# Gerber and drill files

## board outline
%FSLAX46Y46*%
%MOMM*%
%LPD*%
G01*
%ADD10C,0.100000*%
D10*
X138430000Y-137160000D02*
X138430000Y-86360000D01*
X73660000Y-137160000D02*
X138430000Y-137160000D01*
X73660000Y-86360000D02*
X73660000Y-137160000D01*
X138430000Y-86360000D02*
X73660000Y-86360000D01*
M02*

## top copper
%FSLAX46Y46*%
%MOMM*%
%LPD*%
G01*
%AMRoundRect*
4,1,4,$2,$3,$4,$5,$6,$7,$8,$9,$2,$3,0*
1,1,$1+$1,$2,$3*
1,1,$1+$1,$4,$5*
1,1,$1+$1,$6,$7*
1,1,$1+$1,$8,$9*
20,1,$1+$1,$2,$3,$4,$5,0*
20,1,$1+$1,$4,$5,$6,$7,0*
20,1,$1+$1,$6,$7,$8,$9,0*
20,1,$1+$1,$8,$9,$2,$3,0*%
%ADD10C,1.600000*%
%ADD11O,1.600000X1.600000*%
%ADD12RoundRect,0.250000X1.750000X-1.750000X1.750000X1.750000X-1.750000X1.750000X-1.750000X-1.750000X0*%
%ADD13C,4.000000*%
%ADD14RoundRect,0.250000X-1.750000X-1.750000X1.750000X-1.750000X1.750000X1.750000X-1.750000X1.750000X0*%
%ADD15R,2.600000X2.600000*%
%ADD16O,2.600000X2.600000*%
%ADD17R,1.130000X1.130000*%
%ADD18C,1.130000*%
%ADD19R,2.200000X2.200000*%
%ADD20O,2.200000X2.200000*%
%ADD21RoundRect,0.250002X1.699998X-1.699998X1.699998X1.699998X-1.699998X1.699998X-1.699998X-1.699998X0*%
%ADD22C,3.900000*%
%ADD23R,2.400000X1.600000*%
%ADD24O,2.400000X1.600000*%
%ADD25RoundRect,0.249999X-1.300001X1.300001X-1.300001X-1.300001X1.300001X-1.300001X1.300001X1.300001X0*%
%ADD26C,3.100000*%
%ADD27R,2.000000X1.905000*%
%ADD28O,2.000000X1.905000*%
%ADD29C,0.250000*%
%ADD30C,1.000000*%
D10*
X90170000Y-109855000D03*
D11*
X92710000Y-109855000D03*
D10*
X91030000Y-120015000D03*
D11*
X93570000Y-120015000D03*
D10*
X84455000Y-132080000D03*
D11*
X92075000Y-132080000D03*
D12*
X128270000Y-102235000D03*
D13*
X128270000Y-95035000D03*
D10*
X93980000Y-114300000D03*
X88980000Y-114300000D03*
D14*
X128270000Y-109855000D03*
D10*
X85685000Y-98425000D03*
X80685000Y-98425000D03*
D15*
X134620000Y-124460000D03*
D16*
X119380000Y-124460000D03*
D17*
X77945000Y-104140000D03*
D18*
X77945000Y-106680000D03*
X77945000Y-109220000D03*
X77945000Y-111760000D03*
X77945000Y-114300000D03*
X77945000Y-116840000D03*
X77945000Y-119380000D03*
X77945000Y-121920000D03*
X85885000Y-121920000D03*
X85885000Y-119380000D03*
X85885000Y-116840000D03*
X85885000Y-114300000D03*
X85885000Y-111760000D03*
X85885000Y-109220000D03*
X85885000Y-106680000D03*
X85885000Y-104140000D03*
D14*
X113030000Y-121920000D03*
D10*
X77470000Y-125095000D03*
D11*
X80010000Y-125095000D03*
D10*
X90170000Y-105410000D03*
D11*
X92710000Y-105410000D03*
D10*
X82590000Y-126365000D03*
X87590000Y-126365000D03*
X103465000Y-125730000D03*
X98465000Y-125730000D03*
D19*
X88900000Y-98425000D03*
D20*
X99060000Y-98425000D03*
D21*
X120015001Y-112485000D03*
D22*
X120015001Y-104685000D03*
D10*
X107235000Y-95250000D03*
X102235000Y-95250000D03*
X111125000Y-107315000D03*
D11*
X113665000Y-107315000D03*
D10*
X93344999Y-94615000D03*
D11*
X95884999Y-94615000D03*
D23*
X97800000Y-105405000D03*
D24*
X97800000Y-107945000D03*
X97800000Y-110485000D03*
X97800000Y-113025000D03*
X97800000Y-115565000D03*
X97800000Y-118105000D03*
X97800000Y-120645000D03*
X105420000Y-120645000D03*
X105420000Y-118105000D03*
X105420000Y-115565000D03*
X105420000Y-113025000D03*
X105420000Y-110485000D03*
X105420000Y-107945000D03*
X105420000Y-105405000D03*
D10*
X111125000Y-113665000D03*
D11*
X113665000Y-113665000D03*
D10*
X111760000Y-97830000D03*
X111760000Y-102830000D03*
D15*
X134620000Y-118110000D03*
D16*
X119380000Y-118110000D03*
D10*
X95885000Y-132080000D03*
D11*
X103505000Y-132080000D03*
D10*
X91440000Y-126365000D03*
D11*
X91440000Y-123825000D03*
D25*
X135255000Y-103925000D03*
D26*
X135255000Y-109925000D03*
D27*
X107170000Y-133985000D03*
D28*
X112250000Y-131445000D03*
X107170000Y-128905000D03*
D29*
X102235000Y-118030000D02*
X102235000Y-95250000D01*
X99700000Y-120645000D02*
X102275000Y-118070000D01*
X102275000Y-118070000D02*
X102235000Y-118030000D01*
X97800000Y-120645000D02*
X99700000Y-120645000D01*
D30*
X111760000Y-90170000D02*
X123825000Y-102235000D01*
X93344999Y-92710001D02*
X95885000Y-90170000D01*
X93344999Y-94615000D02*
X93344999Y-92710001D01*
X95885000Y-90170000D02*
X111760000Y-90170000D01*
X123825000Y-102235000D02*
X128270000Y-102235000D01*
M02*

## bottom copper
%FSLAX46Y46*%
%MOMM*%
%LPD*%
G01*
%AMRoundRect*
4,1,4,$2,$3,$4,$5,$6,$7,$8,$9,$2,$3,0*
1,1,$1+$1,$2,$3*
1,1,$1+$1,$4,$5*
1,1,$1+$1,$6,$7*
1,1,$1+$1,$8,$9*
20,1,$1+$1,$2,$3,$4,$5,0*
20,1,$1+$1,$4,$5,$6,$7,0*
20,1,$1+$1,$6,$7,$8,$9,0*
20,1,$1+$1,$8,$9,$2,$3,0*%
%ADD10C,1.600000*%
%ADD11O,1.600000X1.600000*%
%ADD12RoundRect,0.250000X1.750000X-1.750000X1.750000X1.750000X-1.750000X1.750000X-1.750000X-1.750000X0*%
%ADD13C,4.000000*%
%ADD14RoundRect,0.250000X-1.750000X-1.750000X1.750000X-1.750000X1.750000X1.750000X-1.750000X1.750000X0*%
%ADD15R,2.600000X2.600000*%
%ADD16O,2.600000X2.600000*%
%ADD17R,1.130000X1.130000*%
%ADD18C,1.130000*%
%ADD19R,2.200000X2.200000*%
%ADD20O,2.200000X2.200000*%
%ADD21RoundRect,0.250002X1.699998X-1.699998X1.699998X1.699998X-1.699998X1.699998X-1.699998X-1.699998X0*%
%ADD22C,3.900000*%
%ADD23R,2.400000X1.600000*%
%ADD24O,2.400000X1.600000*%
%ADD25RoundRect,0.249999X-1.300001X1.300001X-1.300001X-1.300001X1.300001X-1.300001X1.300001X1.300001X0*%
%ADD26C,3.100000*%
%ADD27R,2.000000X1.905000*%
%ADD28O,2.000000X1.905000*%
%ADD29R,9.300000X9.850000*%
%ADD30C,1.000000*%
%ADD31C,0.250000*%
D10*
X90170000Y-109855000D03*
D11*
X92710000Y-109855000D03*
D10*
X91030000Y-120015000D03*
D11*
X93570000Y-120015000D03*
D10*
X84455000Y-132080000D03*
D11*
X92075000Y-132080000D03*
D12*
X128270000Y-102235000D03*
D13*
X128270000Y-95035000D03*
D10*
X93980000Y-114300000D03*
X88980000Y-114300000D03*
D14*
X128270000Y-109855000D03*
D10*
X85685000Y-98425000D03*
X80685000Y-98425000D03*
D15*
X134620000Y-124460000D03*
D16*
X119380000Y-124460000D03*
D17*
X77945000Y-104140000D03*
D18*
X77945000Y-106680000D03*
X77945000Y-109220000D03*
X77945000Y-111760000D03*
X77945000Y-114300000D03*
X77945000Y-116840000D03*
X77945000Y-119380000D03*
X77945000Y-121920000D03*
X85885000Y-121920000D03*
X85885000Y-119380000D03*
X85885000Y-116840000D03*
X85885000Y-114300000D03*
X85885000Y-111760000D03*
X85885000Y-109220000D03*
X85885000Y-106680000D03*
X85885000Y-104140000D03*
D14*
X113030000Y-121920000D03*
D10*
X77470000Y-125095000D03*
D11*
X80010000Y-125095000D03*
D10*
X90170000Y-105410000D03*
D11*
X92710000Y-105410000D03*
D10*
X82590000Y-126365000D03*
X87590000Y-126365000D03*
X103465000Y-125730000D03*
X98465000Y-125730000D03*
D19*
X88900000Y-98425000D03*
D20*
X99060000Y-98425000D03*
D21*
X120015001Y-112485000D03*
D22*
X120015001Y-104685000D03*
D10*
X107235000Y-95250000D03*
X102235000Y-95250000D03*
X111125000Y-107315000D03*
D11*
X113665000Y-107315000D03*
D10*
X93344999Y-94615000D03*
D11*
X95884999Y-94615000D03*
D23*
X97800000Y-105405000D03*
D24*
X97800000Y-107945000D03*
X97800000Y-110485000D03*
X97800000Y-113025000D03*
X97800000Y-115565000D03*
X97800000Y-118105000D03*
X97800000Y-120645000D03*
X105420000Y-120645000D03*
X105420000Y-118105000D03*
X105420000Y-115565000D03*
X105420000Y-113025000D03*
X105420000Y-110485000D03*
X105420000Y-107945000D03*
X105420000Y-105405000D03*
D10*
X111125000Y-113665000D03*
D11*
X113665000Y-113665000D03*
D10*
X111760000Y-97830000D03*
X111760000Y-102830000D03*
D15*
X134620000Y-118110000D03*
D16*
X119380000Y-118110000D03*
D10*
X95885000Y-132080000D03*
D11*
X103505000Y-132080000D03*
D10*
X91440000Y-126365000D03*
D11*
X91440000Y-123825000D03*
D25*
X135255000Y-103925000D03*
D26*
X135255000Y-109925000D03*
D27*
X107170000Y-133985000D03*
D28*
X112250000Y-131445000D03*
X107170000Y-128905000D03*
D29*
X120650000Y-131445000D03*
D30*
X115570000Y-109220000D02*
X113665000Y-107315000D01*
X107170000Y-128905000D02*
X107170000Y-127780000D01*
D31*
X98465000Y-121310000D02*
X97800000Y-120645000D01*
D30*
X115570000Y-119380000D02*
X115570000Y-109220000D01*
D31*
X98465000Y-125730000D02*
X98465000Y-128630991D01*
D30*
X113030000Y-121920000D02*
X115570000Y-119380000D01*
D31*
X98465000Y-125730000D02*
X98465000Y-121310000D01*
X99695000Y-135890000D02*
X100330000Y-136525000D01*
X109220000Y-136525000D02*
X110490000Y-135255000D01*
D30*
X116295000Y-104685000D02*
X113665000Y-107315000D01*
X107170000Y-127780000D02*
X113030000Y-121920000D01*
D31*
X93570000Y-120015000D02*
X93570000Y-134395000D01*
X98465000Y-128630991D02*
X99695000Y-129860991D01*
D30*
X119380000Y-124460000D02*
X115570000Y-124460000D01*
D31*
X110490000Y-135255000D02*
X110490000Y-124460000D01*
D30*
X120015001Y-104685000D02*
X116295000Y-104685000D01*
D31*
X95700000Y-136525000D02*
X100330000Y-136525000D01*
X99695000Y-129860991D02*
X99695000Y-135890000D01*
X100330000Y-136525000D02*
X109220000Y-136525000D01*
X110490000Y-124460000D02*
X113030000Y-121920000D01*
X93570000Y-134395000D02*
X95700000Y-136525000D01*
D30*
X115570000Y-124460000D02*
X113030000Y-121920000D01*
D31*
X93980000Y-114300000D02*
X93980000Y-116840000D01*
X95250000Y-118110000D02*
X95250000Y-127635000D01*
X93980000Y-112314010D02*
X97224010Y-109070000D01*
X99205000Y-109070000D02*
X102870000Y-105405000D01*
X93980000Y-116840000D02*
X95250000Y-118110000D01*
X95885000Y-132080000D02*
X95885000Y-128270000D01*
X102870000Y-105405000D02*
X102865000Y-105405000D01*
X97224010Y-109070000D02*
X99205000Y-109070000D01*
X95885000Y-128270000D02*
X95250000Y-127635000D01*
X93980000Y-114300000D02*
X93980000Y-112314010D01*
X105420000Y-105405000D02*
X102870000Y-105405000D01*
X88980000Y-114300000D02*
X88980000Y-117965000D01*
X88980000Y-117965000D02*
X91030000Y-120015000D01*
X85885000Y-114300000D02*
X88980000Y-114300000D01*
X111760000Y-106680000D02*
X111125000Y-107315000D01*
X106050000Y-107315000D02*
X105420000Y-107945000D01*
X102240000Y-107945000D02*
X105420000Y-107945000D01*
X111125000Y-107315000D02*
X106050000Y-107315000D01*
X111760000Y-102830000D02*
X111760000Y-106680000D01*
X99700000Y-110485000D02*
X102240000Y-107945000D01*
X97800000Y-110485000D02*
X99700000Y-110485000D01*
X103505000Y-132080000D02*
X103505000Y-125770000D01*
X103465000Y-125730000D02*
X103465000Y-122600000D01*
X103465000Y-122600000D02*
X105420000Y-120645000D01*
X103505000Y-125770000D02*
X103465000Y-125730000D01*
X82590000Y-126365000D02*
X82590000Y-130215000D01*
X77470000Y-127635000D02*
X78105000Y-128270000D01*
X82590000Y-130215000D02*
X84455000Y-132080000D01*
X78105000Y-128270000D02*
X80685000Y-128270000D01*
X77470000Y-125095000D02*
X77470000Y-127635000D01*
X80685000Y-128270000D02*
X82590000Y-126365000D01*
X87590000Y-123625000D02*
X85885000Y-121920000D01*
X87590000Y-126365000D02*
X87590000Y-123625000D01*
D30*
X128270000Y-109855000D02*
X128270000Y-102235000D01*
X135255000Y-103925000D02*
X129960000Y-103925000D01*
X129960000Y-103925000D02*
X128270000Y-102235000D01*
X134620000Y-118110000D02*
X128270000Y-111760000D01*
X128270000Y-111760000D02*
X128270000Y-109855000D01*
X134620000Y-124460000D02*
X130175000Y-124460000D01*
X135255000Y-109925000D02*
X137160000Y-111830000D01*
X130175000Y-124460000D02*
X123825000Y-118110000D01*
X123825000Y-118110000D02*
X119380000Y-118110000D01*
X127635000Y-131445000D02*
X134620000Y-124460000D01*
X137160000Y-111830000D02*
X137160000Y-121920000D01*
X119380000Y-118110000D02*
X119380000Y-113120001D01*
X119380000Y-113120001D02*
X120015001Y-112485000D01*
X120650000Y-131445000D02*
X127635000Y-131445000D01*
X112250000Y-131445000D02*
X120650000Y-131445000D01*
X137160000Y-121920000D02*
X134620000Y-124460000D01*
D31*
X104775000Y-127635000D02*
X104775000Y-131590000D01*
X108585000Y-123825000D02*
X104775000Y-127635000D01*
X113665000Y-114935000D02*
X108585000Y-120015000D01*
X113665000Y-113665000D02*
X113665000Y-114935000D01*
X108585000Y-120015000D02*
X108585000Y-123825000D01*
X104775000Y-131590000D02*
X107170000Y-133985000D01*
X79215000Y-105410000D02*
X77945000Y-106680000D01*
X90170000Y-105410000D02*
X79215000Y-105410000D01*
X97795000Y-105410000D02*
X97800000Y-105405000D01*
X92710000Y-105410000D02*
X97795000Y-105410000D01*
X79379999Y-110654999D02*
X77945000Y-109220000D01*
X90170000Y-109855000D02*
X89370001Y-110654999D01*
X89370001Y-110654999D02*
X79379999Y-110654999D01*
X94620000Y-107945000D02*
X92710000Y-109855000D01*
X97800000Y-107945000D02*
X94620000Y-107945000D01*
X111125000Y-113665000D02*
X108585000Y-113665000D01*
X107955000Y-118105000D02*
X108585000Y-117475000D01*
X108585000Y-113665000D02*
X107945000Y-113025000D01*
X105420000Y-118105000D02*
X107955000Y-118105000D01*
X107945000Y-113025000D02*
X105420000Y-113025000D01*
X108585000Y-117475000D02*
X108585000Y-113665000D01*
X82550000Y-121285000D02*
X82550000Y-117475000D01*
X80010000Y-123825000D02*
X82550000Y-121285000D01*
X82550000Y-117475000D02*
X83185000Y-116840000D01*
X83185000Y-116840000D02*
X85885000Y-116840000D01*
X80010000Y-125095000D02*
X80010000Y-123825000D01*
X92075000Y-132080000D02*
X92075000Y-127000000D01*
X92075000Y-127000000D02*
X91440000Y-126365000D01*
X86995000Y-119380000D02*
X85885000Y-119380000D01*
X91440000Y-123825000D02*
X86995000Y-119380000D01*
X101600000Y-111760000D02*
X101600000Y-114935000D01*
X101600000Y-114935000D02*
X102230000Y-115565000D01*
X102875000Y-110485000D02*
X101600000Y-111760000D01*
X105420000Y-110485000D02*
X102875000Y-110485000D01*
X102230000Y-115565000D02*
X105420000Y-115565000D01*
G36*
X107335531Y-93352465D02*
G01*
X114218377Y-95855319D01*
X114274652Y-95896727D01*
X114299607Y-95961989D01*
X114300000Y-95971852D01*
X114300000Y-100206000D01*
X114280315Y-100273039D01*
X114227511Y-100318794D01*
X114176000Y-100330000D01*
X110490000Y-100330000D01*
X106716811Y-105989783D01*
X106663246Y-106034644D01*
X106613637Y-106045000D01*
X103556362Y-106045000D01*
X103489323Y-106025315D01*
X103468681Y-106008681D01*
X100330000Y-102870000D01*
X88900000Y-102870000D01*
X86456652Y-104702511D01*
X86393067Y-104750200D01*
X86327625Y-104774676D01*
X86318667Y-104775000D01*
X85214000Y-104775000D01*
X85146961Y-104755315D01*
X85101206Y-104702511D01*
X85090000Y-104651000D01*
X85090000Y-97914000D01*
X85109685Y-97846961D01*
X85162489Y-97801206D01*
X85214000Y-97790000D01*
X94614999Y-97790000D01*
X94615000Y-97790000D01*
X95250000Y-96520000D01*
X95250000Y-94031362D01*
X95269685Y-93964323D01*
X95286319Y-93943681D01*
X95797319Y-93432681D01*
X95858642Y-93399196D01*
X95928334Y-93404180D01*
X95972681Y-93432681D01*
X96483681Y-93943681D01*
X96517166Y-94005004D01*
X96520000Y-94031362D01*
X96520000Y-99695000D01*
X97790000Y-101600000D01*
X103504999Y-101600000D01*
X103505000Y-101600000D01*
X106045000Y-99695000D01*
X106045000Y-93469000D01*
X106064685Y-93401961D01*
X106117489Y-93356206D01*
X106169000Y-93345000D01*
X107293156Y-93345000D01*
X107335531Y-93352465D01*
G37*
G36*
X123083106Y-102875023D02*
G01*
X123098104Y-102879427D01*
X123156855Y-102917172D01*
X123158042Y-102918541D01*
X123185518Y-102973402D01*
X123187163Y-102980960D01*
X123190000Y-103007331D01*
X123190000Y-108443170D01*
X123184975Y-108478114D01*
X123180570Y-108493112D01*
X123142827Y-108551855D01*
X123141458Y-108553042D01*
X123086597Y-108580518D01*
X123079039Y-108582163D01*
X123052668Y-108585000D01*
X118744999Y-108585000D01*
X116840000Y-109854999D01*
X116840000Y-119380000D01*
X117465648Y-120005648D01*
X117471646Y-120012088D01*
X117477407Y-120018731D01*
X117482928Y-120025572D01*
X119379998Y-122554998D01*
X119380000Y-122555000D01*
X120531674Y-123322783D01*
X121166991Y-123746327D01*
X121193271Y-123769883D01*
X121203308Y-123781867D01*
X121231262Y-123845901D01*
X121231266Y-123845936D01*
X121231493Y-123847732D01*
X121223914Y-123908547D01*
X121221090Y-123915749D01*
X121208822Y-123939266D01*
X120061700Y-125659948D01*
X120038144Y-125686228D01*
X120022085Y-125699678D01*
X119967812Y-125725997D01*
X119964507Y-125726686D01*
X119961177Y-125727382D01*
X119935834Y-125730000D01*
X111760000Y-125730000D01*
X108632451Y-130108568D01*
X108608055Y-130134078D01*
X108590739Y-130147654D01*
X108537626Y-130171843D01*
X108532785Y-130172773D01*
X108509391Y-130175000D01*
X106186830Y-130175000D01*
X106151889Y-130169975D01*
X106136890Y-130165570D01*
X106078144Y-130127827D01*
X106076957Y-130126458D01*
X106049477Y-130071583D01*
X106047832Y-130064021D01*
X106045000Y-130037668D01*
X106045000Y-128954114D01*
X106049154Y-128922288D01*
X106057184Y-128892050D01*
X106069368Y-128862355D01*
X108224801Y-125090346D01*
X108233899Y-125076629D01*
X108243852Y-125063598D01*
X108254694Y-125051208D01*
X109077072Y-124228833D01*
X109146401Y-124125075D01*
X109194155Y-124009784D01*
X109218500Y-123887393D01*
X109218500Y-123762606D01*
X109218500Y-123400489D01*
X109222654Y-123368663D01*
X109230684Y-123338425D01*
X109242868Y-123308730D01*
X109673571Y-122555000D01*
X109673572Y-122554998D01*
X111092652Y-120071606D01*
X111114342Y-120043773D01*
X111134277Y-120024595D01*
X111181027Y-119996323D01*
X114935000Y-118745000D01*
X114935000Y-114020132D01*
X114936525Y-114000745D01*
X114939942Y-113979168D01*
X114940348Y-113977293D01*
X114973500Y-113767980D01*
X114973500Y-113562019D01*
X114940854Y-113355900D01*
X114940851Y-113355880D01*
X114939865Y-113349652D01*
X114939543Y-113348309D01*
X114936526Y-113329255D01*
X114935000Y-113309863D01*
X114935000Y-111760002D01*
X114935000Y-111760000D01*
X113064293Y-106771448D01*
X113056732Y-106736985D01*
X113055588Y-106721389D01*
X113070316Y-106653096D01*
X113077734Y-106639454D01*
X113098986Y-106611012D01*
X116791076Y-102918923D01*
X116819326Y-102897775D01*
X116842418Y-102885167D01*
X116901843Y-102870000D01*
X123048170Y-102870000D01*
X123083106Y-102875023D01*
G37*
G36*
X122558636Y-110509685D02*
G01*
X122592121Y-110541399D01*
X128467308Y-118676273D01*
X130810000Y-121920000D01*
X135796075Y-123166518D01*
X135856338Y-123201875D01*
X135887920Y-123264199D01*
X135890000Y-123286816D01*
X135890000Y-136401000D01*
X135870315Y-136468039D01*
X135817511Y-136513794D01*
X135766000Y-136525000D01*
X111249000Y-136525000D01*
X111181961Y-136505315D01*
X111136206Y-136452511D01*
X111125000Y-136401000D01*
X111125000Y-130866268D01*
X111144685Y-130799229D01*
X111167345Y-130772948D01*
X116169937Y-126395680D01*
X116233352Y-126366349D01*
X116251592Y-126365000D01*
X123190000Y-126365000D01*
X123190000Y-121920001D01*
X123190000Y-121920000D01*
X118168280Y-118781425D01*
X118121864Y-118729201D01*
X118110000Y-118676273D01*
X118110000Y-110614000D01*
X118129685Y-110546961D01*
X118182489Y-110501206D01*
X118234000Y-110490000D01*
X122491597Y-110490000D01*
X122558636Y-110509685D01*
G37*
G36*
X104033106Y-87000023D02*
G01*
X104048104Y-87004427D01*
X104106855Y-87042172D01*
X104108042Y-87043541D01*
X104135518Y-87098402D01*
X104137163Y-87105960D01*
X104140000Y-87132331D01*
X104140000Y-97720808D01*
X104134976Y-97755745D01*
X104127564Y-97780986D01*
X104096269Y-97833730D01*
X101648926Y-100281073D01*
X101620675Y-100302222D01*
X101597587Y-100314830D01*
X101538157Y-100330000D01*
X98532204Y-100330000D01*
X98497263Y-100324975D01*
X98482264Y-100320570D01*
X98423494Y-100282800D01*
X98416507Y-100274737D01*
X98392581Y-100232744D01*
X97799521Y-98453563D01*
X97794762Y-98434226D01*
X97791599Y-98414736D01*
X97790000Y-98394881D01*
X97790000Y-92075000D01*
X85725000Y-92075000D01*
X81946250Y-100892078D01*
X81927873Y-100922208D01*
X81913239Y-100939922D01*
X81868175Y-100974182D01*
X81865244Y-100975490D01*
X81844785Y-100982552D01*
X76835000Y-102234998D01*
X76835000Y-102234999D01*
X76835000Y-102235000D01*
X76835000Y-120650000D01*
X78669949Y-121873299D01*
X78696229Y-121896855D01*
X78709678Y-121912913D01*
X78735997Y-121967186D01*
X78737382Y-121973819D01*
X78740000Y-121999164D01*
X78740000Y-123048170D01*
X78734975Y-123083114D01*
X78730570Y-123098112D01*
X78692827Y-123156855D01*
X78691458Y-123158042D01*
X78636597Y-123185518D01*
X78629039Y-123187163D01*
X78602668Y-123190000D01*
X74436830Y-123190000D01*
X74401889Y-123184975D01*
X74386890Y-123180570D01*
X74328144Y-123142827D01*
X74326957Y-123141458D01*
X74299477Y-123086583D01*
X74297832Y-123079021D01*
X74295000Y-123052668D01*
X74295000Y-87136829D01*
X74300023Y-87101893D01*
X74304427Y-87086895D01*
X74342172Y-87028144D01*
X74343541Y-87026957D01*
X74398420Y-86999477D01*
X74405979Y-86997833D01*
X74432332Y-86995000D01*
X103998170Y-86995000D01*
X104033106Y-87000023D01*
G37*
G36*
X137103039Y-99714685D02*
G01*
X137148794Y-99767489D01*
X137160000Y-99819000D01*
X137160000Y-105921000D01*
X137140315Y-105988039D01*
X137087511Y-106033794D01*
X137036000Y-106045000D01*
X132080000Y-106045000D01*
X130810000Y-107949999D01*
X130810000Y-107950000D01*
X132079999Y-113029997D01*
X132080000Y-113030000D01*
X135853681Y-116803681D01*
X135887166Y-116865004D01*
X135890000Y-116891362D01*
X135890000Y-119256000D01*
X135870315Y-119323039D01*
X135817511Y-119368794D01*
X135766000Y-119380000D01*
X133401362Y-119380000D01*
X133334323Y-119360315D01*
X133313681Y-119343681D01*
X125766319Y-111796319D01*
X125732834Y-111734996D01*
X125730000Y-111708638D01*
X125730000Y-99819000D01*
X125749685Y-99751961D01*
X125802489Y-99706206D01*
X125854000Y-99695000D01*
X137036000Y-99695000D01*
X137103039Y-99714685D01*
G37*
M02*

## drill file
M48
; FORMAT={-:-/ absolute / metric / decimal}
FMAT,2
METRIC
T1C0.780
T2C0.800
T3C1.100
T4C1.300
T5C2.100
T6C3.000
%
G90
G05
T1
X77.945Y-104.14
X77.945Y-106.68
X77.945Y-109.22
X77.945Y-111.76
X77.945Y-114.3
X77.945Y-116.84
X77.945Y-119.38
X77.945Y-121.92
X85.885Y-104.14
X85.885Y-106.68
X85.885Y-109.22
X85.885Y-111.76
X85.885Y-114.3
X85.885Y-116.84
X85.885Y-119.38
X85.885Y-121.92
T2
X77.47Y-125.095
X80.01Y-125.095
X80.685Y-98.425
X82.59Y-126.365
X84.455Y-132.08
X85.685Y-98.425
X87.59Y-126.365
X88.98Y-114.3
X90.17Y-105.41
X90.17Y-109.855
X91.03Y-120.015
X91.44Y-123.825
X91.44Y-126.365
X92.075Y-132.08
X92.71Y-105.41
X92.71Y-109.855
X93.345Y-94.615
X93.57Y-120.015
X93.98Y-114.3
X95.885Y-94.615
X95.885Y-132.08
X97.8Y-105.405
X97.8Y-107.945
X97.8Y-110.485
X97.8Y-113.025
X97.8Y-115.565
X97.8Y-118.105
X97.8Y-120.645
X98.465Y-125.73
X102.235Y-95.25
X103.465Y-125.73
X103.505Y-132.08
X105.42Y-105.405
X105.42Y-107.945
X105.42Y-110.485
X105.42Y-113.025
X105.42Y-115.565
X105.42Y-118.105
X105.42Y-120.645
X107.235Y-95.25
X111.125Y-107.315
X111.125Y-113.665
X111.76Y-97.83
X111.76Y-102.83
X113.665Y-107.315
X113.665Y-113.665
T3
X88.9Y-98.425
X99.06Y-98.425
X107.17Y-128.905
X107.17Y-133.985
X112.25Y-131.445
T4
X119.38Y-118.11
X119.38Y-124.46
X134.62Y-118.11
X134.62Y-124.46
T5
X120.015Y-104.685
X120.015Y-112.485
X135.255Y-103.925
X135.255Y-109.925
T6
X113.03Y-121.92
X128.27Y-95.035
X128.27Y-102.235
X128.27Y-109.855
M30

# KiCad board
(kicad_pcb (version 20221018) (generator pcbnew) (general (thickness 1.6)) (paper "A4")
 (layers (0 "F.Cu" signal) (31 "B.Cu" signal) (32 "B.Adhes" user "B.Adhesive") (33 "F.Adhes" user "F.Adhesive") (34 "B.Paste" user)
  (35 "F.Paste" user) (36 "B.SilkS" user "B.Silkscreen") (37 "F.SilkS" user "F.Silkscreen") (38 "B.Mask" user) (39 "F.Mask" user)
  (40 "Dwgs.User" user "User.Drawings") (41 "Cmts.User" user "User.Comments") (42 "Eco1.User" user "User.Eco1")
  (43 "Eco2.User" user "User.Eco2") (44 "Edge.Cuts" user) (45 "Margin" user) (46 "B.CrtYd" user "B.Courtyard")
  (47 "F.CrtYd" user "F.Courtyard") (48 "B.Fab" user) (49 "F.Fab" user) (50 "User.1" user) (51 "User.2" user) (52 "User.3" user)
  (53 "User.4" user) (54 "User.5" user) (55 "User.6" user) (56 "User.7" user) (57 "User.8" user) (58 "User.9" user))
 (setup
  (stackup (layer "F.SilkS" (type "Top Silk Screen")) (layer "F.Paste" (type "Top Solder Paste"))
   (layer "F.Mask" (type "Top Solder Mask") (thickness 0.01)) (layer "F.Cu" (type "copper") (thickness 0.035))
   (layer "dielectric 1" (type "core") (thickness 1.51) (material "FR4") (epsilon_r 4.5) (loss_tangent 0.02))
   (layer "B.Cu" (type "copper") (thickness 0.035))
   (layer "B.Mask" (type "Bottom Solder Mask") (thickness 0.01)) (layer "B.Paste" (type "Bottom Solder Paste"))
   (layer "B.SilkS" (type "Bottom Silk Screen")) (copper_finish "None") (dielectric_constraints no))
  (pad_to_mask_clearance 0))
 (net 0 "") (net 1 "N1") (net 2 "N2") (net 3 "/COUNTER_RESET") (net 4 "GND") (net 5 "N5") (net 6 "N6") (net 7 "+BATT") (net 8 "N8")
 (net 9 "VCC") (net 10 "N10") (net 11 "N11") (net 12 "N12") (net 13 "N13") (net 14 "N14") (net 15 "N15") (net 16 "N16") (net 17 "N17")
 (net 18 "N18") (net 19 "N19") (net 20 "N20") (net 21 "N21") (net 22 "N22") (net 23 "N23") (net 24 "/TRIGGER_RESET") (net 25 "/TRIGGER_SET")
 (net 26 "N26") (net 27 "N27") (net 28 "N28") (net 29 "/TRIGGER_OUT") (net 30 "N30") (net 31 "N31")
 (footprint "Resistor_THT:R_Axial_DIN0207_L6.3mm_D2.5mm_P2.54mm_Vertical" (layer "F.Cu") (at 90.17 109.855)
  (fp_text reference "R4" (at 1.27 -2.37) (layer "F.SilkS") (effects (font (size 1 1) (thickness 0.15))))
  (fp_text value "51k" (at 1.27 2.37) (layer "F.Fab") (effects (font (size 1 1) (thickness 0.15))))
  (pad "1" thru_hole circle (at 0 0) (size 1.6 1.6) (drill 0.8) (layers "*.Cu" "*.Mask") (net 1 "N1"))
  (pad "2" thru_hole oval (at 2.54 0) (size 1.6 1.6) (drill 0.8) (layers "*.Cu" "*.Mask") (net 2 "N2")))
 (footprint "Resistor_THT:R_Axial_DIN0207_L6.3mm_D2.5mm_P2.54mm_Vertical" (layer "F.Cu") (at 91.03 120.015)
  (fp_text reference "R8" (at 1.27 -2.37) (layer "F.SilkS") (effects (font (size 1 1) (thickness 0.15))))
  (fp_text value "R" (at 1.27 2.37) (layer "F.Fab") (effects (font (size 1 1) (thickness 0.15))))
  (pad "1" thru_hole circle (at 0 0) (size 1.6 1.6) (drill 0.8) (layers "*.Cu" "*.Mask") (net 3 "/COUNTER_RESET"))
  (pad "2" thru_hole oval (at 2.54 0) (size 1.6 1.6) (drill 0.8) (layers "*.Cu" "*.Mask") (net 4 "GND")))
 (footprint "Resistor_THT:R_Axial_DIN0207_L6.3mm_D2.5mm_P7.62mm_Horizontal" (layer "F.Cu") (at 84.455 132.08)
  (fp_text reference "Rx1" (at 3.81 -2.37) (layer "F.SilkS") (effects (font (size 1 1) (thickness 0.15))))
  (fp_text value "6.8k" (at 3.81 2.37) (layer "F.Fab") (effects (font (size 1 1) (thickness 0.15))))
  (pad "1" thru_hole circle (at 0 0) (size 1.6 1.6) (drill 0.8) (layers "*.Cu" "*.Mask") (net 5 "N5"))
  (pad "2" thru_hole oval (at 7.62 0) (size 1.6 1.6) (drill 0.8) (layers "*.Cu" "*.Mask") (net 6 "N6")))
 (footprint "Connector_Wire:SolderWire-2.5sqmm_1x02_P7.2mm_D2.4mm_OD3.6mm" (layer "F.Cu") (at 128.27 102.235 90)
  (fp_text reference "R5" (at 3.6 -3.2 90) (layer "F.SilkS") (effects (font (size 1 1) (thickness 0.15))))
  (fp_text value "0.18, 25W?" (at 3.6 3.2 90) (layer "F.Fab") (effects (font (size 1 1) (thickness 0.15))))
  (pad "1" thru_hole roundrect (at 0 0 90) (size 4 4) (drill 3) (layers "*.Cu" "*.Mask") (roundrect_rratio 0.0625) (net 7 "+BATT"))
  (pad "2" thru_hole circle (at 7.2 0 90) (size 4 4) (drill 3) (layers "*.Cu" "*.Mask") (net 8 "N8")))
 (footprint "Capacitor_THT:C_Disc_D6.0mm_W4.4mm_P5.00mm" (layer "F.Cu") (at 93.98 114.3 180)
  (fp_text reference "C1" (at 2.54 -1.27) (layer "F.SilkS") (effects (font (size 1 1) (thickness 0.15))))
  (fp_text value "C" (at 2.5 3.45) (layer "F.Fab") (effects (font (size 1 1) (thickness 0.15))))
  (pad "1" thru_hole circle (at 0 0 180) (size 1.6 1.6) (drill 0.8) (layers "*.Cu" "*.Mask") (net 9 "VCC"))
  (pad "2" thru_hole circle (at 5 0 180) (size 1.6 1.6) (drill 0.8) (layers "*.Cu" "*.Mask") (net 3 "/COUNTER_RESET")))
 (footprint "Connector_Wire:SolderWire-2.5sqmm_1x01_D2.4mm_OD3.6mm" (layer "F.Cu") (at 128.27 109.855)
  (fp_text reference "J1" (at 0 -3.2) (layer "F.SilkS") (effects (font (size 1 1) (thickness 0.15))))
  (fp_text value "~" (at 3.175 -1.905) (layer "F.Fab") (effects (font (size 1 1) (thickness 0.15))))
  (pad "1" thru_hole roundrect (at 0 0) (size 4 4) (drill 3) (layers "*.Cu" "*.Mask") (roundrect_rratio 0.0625) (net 7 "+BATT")))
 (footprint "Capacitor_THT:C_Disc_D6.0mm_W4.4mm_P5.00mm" (layer "F.Cu") (at 85.685 98.425 180)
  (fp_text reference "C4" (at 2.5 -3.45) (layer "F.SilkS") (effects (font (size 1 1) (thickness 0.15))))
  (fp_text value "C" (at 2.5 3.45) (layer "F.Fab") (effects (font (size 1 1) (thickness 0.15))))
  (pad "1" thru_hole circle (at 0 0 180) (size 1.6 1.6) (drill 0.8) (layers "*.Cu" "*.Mask") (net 9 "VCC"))
  (pad "2" thru_hole circle (at 5 0 180) (size 1.6 1.6) (drill 0.8) (layers "*.Cu" "*.Mask") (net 4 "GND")))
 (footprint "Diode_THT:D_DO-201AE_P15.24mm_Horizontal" (layer "F.Cu") (at 134.62 124.46 180)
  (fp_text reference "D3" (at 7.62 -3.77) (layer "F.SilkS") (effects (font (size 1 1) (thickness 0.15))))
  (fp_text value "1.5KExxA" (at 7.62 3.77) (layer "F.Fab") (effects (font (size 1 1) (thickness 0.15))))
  (pad "1" thru_hole rect (at 0 0 180) (size 2.6 2.6) (drill 1.3) (layers "*.Cu" "*.Mask") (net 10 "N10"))
  (pad "2" thru_hole oval (at 15.24 0 180) (size 2.6 2.6) (drill 1.3) (layers "*.Cu" "*.Mask") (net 4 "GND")))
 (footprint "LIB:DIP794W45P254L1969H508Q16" (layer "F.Cu") (at 81.915 113.03)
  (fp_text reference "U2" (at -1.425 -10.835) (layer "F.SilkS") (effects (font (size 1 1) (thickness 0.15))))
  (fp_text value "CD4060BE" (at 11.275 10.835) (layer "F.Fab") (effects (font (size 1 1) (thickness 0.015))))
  (pad "1" thru_hole rect (at -3.97 -8.89) (size 1.13 1.13) (drill 0.78) (layers "*.Cu" "*.Mask") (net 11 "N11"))
  (pad "2" thru_hole circle (at -3.97 -6.35) (size 1.13 1.13) (drill 0.78) (layers "*.Cu" "*.Mask") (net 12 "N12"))
  (pad "3" thru_hole circle (at -3.97 -3.81) (size 1.13 1.13) (drill 0.78) (layers "*.Cu" "*.Mask") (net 1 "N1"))
  (pad "4" thru_hole circle (at -3.97 -1.27) (size 1.13 1.13) (drill 0.78) (layers "*.Cu" "*.Mask") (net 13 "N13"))
  (pad "5" thru_hole circle (at -3.97 1.27) (size 1.13 1.13) (drill 0.78) (layers "*.Cu" "*.Mask") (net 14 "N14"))
  (pad "6" thru_hole circle (at -3.97 3.81) (size 1.13 1.13) (drill 0.78) (layers "*.Cu" "*.Mask") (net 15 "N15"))
  (pad "7" thru_hole circle (at -3.97 6.35) (size 1.13 1.13) (drill 0.78) (layers "*.Cu" "*.Mask") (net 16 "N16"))
  (pad "8" thru_hole circle (at -3.97 8.89) (size 1.13 1.13) (drill 0.78) (layers "*.Cu" "*.Mask") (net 4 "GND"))
  (pad "9" thru_hole circle (at 3.97 8.89) (size 1.13 1.13) (drill 0.78) (layers "*.Cu" "*.Mask") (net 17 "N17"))
  (pad "10" thru_hole circle (at 3.97 6.35) (size 1.13 1.13) (drill 0.78) (layers "*.Cu" "*.Mask") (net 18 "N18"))
  (pad "11" thru_hole circle (at 3.97 3.81) (size 1.13 1.13) (drill 0.78) (layers "*.Cu" "*.Mask") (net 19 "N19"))
  (pad "12" thru_hole circle (at 3.97 1.27) (size 1.13 1.13) (drill 0.78) (layers "*.Cu" "*.Mask") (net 3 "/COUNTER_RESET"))
  (pad "13" thru_hole circle (at 3.97 -1.27) (size 1.13 1.13) (drill 0.78) (layers "*.Cu" "*.Mask") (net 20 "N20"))
  (pad "14" thru_hole circle (at 3.97 -3.81) (size 1.13 1.13) (drill 0.78) (layers "*.Cu" "*.Mask") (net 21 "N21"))
  (pad "15" thru_hole circle (at 3.97 -6.35) (size 1.13 1.13) (drill 0.78) (layers "*.Cu" "*.Mask") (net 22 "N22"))
  (pad "16" thru_hole circle (at 3.97 -8.89) (size 1.13 1.13) (drill 0.78) (layers "*.Cu" "*.Mask") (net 9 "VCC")))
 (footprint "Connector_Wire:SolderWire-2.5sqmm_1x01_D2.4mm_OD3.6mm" (layer "F.Cu") (at 113.03 121.92)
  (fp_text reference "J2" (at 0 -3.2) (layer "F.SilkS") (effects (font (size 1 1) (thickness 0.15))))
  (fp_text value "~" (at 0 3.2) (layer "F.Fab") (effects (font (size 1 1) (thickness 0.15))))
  (pad "1" thru_hole roundrect (at 0 0) (size 4 4) (drill 3) (layers "*.Cu" "*.Mask") (roundrect_rratio 0.0625) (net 4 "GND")))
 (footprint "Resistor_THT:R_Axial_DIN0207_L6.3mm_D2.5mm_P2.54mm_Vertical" (layer "F.Cu") (at 77.47 125.095)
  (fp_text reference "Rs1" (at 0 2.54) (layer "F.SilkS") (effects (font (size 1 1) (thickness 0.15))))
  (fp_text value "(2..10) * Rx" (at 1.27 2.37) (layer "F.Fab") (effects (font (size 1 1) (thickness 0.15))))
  (pad "1" thru_hole circle (at 0 0) (size 1.6 1.6) (drill 0.8) (layers "*.Cu" "*.Mask") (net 5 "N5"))
  (pad "2" thru_hole oval (at 2.54 0) (size 1.6 1.6) (drill 0.8) (layers "*.Cu" "*.Mask") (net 19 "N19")))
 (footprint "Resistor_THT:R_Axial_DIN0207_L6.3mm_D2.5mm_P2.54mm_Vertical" (layer "F.Cu") (at 90.17 105.41)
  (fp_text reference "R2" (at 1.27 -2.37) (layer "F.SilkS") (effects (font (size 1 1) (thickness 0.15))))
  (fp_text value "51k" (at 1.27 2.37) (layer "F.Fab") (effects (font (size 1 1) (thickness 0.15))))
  (pad "1" thru_hole circle (at 0 0) (size 1.6 1.6) (drill 0.8) (layers "*.Cu" "*.Mask") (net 12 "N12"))
  (pad "2" thru_hole oval (at 2.54 0) (size 1.6 1.6) (drill 0.8) (layers "*.Cu" "*.Mask") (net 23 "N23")))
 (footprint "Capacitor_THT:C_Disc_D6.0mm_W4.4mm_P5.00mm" (layer "F.Cu") (at 82.59 126.365)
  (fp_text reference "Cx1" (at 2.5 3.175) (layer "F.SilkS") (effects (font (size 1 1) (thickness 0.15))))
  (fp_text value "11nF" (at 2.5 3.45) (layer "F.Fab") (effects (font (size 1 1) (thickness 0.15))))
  (pad "1" thru_hole circle (at 0 0) (size 1.6 1.6) (drill 0.8) (layers "*.Cu" "*.Mask") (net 5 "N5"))
  (pad "2" thru_hole circle (at 5 0) (size 1.6 1.6) (drill 0.8) (layers "*.Cu" "*.Mask") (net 17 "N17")))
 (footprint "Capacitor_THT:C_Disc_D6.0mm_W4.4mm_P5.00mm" (layer "F.Cu") (at 103.465 125.73 180)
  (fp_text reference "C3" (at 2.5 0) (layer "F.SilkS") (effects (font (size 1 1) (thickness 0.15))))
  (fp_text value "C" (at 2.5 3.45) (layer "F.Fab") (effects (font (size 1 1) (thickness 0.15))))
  (pad "1" thru_hole circle (at 0 0 180) (size 1.6 1.6) (drill 0.8) (layers "*.Cu" "*.Mask") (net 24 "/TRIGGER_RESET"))
  (pad "2" thru_hole circle (at 5 0 180) (size 1.6 1.6) (drill 0.8) (layers "*.Cu" "*.Mask") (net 4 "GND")))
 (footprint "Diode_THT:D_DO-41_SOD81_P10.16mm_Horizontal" (layer "F.Cu") (at 88.9 98.425)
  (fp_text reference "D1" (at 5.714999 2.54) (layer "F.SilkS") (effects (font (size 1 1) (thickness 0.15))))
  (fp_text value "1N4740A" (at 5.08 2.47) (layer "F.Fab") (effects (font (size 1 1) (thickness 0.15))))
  (pad "1" thru_hole rect (at 0 0) (size 2.2 2.2) (drill 1.1) (layers "*.Cu" "*.Mask") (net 9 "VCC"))
  (pad "2" thru_hole oval (at 10.16 0) (size 2.2 2.2) (drill 1.1) (layers "*.Cu" "*.Mask") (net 4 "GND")))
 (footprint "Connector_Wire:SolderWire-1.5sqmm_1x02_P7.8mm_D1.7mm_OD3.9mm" (layer "F.Cu") (at 120.015001 112.485 90)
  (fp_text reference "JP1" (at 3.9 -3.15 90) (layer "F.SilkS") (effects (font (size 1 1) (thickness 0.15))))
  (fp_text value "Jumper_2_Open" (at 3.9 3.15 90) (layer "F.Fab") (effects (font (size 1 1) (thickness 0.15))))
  (pad "1" thru_hole roundrect (at 0 0 90) (size 3.9 3.9) (drill 2.1) (layers "*.Cu" "*.Mask") (roundrect_rratio 0.064103) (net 10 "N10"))
  (pad "2" thru_hole circle (at 7.8 0 90) (size 3.9 3.9) (drill 2.1) (layers "*.Cu" "*.Mask") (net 4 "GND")))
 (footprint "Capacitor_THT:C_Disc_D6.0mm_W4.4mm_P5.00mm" (layer "F.Cu") (at 107.235 95.25 180)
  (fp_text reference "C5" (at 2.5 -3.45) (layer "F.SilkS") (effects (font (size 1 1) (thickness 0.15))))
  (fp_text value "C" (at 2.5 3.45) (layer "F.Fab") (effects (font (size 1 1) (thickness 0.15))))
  (pad "1" thru_hole circle (at 0 0 180) (size 1.6 1.6) (drill 0.8) (layers "*.Cu" "*.Mask") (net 9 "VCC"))
  (pad "2" thru_hole circle (at 5 0 180) (size 1.6 1.6) (drill 0.8) (layers "*.Cu" "*.Mask") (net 4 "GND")))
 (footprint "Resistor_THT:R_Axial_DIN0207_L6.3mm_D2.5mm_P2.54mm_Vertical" (layer "F.Cu") (at 111.125 107.315)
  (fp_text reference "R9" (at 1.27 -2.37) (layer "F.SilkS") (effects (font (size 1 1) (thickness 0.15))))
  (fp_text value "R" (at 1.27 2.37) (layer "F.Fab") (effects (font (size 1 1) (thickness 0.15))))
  (pad "1" thru_hole circle (at 0 0) (size 1.6 1.6) (drill 0.8) (layers "*.Cu" "*.Mask") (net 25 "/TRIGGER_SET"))
  (pad "2" thru_hole oval (at 2.54 0) (size 1.6 1.6) (drill 0.8) (layers "*.Cu" "*.Mask") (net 4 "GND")))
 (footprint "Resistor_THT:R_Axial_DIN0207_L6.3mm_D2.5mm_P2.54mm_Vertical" (layer "F.Cu") (at 93.344999 94.615)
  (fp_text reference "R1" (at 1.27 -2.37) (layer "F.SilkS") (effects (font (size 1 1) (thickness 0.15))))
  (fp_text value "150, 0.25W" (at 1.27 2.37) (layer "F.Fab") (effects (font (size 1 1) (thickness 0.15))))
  (pad "1" thru_hole circle (at 0 0) (size 1.6 1.6) (drill 0.8) (layers "*.Cu" "*.Mask") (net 7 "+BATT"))
  (pad "2" thru_hole oval (at 2.54 0) (size 1.6 1.6) (drill 0.8) (layers "*.Cu" "*.Mask") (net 9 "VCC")))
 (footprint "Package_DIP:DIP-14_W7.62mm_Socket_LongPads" (layer "F.Cu") (at 97.8 105.405)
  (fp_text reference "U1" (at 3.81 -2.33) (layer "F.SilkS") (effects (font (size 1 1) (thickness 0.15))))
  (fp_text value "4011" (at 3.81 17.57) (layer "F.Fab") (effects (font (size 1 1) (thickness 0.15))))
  (pad "1" thru_hole rect (at 0 0) (size 2.4 1.6) (drill 0.8) (layers "*.Cu" "*.Mask") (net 23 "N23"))
  (pad "2" thru_hole oval (at 0 2.54) (size 2.4 1.6) (drill 0.8) (layers "*.Cu" "*.Mask") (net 2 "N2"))
  (pad "3" thru_hole oval (at 0 5.08) (size 2.4 1.6) (drill 0.8) (layers "*.Cu" "*.Mask") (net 25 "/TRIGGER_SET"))
  (pad "4" thru_hole oval (at 0 7.62) (size 2.4 1.6) (drill 0.8) (layers "*.Cu" "*.Mask") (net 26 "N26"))
  (pad "5" thru_hole oval (at 0 10.16) (size 2.4 1.6) (drill 0.8) (layers "*.Cu" "*.Mask") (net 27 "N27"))
  (pad "6" thru_hole oval (at 0 12.7) (size 2.4 1.6) (drill 0.8) (layers "*.Cu" "*.Mask") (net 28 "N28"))
  (pad "7" thru_hole oval (at 0 15.24) (size 2.4 1.6) (drill 0.8) (layers "*.Cu" "*.Mask") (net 4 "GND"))
  (pad "8" thru_hole oval (at 7.62 15.24) (size 2.4 1.6) (drill 0.8) (layers "*.Cu" "*.Mask") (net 24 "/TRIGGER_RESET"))
  (pad "9" thru_hole oval (at 7.62 12.7) (size 2.4 1.6) (drill 0.8) (layers "*.Cu" "*.Mask") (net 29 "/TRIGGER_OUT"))
  (pad "10" thru_hole oval (at 7.62 10.16) (size 2.4 1.6) (drill 0.8) (layers "*.Cu" "*.Mask") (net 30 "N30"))
  (pad "11" thru_hole oval (at 7.62 7.62) (size 2.4 1.6) (drill 0.8) (layers "*.Cu" "*.Mask") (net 29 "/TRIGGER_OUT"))
  (pad "12" thru_hole oval (at 7.62 5.08) (size 2.4 1.6) (drill 0.8) (layers "*.Cu" "*.Mask") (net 30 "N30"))
  (pad "13" thru_hole oval (at 7.62 2.54) (size 2.4 1.6) (drill 0.8) (layers "*.Cu" "*.Mask") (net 25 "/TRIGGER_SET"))
  (pad "14" thru_hole oval (at 7.62 0) (size 2.4 1.6) (drill 0.8) (layers "*.Cu" "*.Mask") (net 9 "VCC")))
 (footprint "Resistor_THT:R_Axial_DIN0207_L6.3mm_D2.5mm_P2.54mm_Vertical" (layer "F.Cu") (at 111.125 113.665)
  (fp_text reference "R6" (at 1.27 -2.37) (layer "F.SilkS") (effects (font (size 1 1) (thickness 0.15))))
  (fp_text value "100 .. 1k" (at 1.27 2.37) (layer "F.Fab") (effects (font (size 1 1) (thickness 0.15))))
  (pad "1" thru_hole circle (at 0 0) (size 1.6 1.6) (drill 0.8) (layers "*.Cu" "*.Mask") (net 29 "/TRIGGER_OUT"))
  (pad "2" thru_hole oval (at 2.54 0) (size 1.6 1.6) (drill 0.8) (layers "*.Cu" "*.Mask") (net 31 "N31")))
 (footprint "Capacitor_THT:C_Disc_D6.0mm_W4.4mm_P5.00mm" (layer "F.Cu") (at 111.76 97.83 -90)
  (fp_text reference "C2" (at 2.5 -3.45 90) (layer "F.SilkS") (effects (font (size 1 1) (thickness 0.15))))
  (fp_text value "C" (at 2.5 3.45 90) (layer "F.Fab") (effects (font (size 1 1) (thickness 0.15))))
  (pad "1" thru_hole circle (at 0 0 270) (size 1.6 1.6) (drill 0.8) (layers "*.Cu" "*.Mask") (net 9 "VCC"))
  (pad "2" thru_hole circle (at 5 0 270) (size 1.6 1.6) (drill 0.8) (layers "*.Cu" "*.Mask") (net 25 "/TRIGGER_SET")))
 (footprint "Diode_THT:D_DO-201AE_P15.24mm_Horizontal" (layer "F.Cu") (at 134.62 118.11 180)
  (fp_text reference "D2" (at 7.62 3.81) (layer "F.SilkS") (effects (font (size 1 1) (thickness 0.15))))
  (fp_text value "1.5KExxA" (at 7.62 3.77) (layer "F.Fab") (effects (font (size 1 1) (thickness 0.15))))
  (pad "1" thru_hole rect (at 0 0 180) (size 2.6 2.6) (drill 1.3) (layers "*.Cu" "*.Mask") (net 7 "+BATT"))
  (pad "2" thru_hole oval (at 15.24 0 180) (size 2.6 2.6) (drill 1.3) (layers "*.Cu" "*.Mask") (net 10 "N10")))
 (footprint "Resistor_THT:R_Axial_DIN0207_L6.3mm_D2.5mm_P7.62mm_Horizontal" (layer "F.Cu") (at 95.885 132.08)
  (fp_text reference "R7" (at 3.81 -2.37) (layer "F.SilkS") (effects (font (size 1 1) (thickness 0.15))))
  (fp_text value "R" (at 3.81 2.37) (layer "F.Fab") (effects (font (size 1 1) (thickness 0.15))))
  (pad "1" thru_hole circle (at 0 0) (size 1.6 1.6) (drill 0.8) (layers "*.Cu" "*.Mask") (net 9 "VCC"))
  (pad "2" thru_hole oval (at 7.62 0) (size 1.6 1.6) (drill 0.8) (layers "*.Cu" "*.Mask") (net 24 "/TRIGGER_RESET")))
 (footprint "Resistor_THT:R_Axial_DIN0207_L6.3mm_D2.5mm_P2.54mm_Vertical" (layer "F.Cu") (at 91.44 126.365 90)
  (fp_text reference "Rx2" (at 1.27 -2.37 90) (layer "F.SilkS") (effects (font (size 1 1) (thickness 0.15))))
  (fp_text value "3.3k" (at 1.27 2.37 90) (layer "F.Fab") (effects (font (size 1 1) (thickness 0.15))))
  (pad "1" thru_hole circle (at 0 0 90) (size 1.6 1.6) (drill 0.8) (layers "*.Cu" "*.Mask") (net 6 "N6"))
  (pad "2" thru_hole oval (at 2.54 0 90) (size 1.6 1.6) (drill 0.8) (layers "*.Cu" "*.Mask") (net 18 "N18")))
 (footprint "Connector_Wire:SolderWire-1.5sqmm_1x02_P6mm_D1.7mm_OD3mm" (layer "F.Cu") (at 135.255 103.925 -90)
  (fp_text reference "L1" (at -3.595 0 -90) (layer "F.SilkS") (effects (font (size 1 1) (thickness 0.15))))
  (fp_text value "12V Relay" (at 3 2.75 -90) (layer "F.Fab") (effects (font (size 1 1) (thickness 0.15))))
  (pad "1" thru_hole roundrect (at 0 0 270) (size 3.1 3.1) (drill 2.1) (layers "*.Cu" "*.Mask") (roundrect_rratio 0.080645) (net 7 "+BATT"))
  (pad "2" thru_hole circle (at 6 0 270) (size 3.1 3.1) (drill 2.1) (layers "*.Cu" "*.Mask") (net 10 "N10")))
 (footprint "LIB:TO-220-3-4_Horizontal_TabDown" (layer "B.Cu") (at 112.25 133.985 90)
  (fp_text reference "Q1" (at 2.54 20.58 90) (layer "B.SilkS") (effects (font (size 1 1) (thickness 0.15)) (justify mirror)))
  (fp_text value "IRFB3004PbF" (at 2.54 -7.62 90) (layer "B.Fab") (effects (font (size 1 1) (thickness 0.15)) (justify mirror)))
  (pad "1" thru_hole rect (at 0 -5.08 90) (size 1.905 2) (drill 1.1) (layers "*.Cu" "*.Mask") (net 31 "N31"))
  (pad "2" thru_hole oval (at 2.54 0 90) (size 1.905 2) (drill 1.1) (layers "*.Cu" "*.Mask") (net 10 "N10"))
  (pad "3" thru_hole oval (at 5.08 -5.08 90) (size 1.905 2) (drill 1.1) (layers "*.Cu" "*.Mask") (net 4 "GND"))
  (pad "4" connect rect (at 2.54 8.4 90) (size 9.85 9.3) (layers "B.Cu" "B.Mask") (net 10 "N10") (zone_connect 2)))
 (gr_line (start 138.43 137.16) (end 138.43 86.36) (stroke (width 0.1) (type default)) (layer "Edge.Cuts"))
 (gr_line (start 73.66 137.16) (end 138.43 137.16) (stroke (width 0.1) (type default)) (layer "Edge.Cuts"))
 (gr_line (start 73.66 86.36) (end 73.66 137.16) (stroke (width 0.1) (type default)) (layer "Edge.Cuts"))
 (gr_line (start 138.43 86.36) (end 73.66 86.36) (stroke (width 0.1) (type default)) (layer "Edge.Cuts"))
 (segment (start 102.235 118.03) (end 102.235 95.25) (width 0.25) (layer "F.Cu") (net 4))
 (segment (start 99.7 120.645) (end 102.275 118.07) (width 0.25) (layer "F.Cu") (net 4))
 (segment (start 102.275 118.07) (end 102.235 118.03) (width 0.25) (layer "F.Cu") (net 4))
 (segment (start 97.8 120.645) (end 99.7 120.645) (width 0.25) (layer "F.Cu") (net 4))
 (segment (start 115.57 109.22) (end 113.665 107.315) (width 1) (layer "B.Cu") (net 4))
 (segment (start 107.17 128.905) (end 107.17 127.78) (width 1) (layer "B.Cu") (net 4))
 (segment (start 98.465 121.31) (end 97.8 120.645) (width 0.25) (layer "B.Cu") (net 4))
 (segment (start 115.57 119.38) (end 115.57 109.22) (width 1) (layer "B.Cu") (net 4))
 (segment (start 98.465 125.73) (end 98.465 128.630991) (width 0.25) (layer "B.Cu") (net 4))
 (segment (start 113.03 121.92) (end 115.57 119.38) (width 1) (layer "B.Cu") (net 4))
 (segment (start 98.465 125.73) (end 98.465 121.31) (width 0.25) (layer "B.Cu") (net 4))
 (segment (start 99.695 135.89) (end 100.33 136.525) (width 0.25) (layer "B.Cu") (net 4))
 (segment (start 109.22 136.525) (end 110.49 135.255) (width 0.25) (layer "B.Cu") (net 4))
 (segment (start 116.295 104.685) (end 113.665 107.315) (width 1) (layer "B.Cu") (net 4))
 (segment (start 107.17 127.78) (end 113.03 121.92) (width 1) (layer "B.Cu") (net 4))
 (segment (start 93.57 120.015) (end 93.57 134.395) (width 0.25) (layer "B.Cu") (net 4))
 (segment (start 98.465 128.630991) (end 99.695 129.860991) (width 0.25) (layer "B.Cu") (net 4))
 (segment (start 119.38 124.46) (end 115.57 124.46) (width 1) (layer "B.Cu") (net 4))
 (segment (start 110.49 135.255) (end 110.49 124.46) (width 0.25) (layer "B.Cu") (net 4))
 (segment (start 120.015001 104.685) (end 116.295 104.685) (width 1) (layer "B.Cu") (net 4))
 (segment (start 95.7 136.525) (end 100.33 136.525) (width 0.25) (layer "B.Cu") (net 4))
 (segment (start 99.695 129.860991) (end 99.695 135.89) (width 0.25) (layer "B.Cu") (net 4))
 (segment (start 100.33 136.525) (end 109.22 136.525) (width 0.25) (layer "B.Cu") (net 4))
 (segment (start 110.49 124.46) (end 113.03 121.92) (width 0.25) (layer "B.Cu") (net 4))
 (segment (start 93.57 134.395) (end 95.7 136.525) (width 0.25) (layer "B.Cu") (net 4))
 (segment (start 115.57 124.46) (end 113.03 121.92) (width 1) (layer "B.Cu") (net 4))
 (segment (start 93.98 114.3) (end 93.98 116.84) (width 0.25) (layer "B.Cu") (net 9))
 (segment (start 95.25 118.11) (end 95.25 127.635) (width 0.25) (layer "B.Cu") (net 9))
 (segment (start 93.98 112.31401) (end 97.22401 109.07) (width 0.25) (layer "B.Cu") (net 9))
 (segment (start 99.205 109.07) (end 102.87 105.405) (width 0.25) (layer "B.Cu") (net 9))
 (segment (start 93.98 116.84) (end 95.25 118.11) (width 0.25) (layer "B.Cu") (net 9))
 (segment (start 95.885 132.08) (end 95.885 128.27) (width 0.25) (layer "B.Cu") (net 9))
 (segment (start 102.87 105.405) (end 102.865 105.405) (width 0.25) (layer "B.Cu") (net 9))
 (segment (start 97.22401 109.07) (end 99.205 109.07) (width 0.25) (layer "B.Cu") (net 9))
 (segment (start 95.885 128.27) (end 95.25 127.635) (width 0.25) (layer "B.Cu") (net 9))
 (segment (start 93.98 114.3) (end 93.98 112.31401) (width 0.25) (layer "B.Cu") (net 9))
 (segment (start 105.42 105.405) (end 102.87 105.405) (width 0.25) (layer "B.Cu") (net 9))
 (segment (start 88.98 114.3) (end 88.98 117.965) (width 0.25) (layer "B.Cu") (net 3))
 (segment (start 88.98 117.965) (end 91.03 120.015) (width 0.25) (layer "B.Cu") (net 3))
 (segment (start 85.885 114.3) (end 88.98 114.3) (width 0.25) (layer "B.Cu") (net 3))
 (segment (start 111.76 106.68) (end 111.125 107.315) (width 0.25) (layer "B.Cu") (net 25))
 (segment (start 106.05 107.315) (end 105.42 107.945) (width 0.25) (layer "B.Cu") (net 25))
 (segment (start 102.24 107.945) (end 105.42 107.945) (width 0.25) (layer "B.Cu") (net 25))
 (segment (start 111.125 107.315) (end 106.05 107.315) (width 0.25) (layer "B.Cu") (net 25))
 (segment (start 111.76 102.83) (end 111.76 106.68) (width 0.25) (layer "B.Cu") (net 25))
 (segment (start 99.7 110.485) (end 102.24 107.945) (width 0.25) (layer "B.Cu") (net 25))
 (segment (start 97.8 110.485) (end 99.7 110.485) (width 0.25) (layer "B.Cu") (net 25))
 (segment (start 103.505 132.08) (end 103.505 125.77) (width 0.25) (layer "B.Cu") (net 24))
 (segment (start 103.465 125.73) (end 103.465 122.6) (width 0.25) (layer "B.Cu") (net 24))
 (segment (start 103.465 122.6) (end 105.42 120.645) (width 0.25) (layer "B.Cu") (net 24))
 (segment (start 103.505 125.77) (end 103.465 125.73) (width 0.25) (layer "B.Cu") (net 24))
 (segment (start 82.59 126.365) (end 82.59 130.215) (width 0.25) (layer "B.Cu") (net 5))
 (segment (start 77.47 127.635) (end 78.105 128.27) (width 0.25) (layer "B.Cu") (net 5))
 (segment (start 82.59 130.215) (end 84.455 132.08) (width 0.25) (layer "B.Cu") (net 5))
 (segment (start 78.105 128.27) (end 80.685 128.27) (width 0.25) (layer "B.Cu") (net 5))
 (segment (start 77.47 125.095) (end 77.47 127.635) (width 0.25) (layer "B.Cu") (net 5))
 (segment (start 80.685 128.27) (end 82.59 126.365) (width 0.25) (layer "B.Cu") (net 5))
 (segment (start 87.59 123.625) (end 85.885 121.92) (width 0.25) (layer "B.Cu") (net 17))
 (segment (start 87.59 126.365) (end 87.59 123.625) (width 0.25) (layer "B.Cu") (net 17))
 (segment (start 111.76 90.17) (end 123.825 102.235) (width 1) (layer "F.Cu") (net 7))
 (segment (start 93.344999 92.710001) (end 95.885 90.17) (width 1) (layer "F.Cu") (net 7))
 (segment (start 93.344999 94.615) (end 93.344999 92.710001) (width 1) (layer "F.Cu") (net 7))
 (segment (start 95.885 90.17) (end 111.76 90.17) (width 1) (layer "F.Cu") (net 7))
 (segment (start 123.825 102.235) (end 128.27 102.235) (width 1) (layer "F.Cu") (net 7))
 (segment (start 128.27 109.855) (end 128.27 102.235) (width 1) (layer "B.Cu") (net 7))
 (segment (start 135.255 103.925) (end 129.96 103.925) (width 1) (layer "B.Cu") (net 7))
 (segment (start 129.96 103.925) (end 128.27 102.235) (width 1) (layer "B.Cu") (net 7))
 (segment (start 134.62 118.11) (end 128.27 111.76) (width 1) (layer "B.Cu") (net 7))
 (segment (start 128.27 111.76) (end 128.27 109.855) (width 1) (layer "B.Cu") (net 7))
 (segment (start 134.62 124.46) (end 130.175 124.46) (width 1) (layer "B.Cu") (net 10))
 (segment (start 135.255 109.925) (end 137.16 111.83) (width 1) (layer "B.Cu") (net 10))
 (segment (start 130.175 124.46) (end 123.825 118.11) (width 1) (layer "B.Cu") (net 10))
 (segment (start 123.825 118.11) (end 119.38 118.11) (width 1) (layer "B.Cu") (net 10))
 (segment (start 127.635 131.445) (end 134.62 124.46) (width 1) (layer "B.Cu") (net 10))
 (segment (start 137.16 111.83) (end 137.16 121.92) (width 1) (layer "B.Cu") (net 10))
 (segment (start 119.38 118.11) (end 119.38 113.120001) (width 1) (layer "B.Cu") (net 10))
 (segment (start 119.38 113.120001) (end 120.015001 112.485) (width 1) (layer "B.Cu") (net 10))
 (segment (start 120.65 131.445) (end 127.635 131.445) (width 1) (layer "B.Cu") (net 10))
 (segment (start 112.25 131.445) (end 120.65 131.445) (width 1) (layer "B.Cu") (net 10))
 (segment (start 137.16 121.92) (end 134.62 124.46) (width 1) (layer "B.Cu") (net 10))
 (segment (start 104.775 127.635) (end 104.775 131.59) (width 0.25) (layer "B.Cu") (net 31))
 (segment (start 108.585 123.825) (end 104.775 127.635) (width 0.25) (layer "B.Cu") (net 31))
 (segment (start 113.665 114.935) (end 108.585 120.015) (width 0.25) (layer "B.Cu") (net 31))
 (segment (start 113.665 113.665) (end 113.665 114.935) (width 0.25) (layer "B.Cu") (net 31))
 (segment (start 108.585 120.015) (end 108.585 123.825) (width 0.25) (layer "B.Cu") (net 31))
 (segment (start 104.775 131.59) (end 107.17 133.985) (width 0.25) (layer "B.Cu") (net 31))
 (segment (start 79.215 105.41) (end 77.945 106.68) (width 0.25) (layer "B.Cu") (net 12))
 (segment (start 90.17 105.41) (end 79.215 105.41) (width 0.25) (layer "B.Cu") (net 12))
 (segment (start 97.795 105.41) (end 97.8 105.405) (width 0.25) (layer "B.Cu") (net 23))
 (segment (start 92.71 105.41) (end 97.795 105.41) (width 0.25) (layer "B.Cu") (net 23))
 (segment (start 79.379999 110.654999) (end 77.945 109.22) (width 0.25) (layer "B.Cu") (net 1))
 (segment (start 90.17 109.855) (end 89.370001 110.654999) (width 0.25) (layer "B.Cu") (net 1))
 (segment (start 89.370001 110.654999) (end 79.379999 110.654999) (width 0.25) (layer "B.Cu") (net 1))
 (segment (start 94.62 107.945) (end 92.71 109.855) (width 0.25) (layer "B.Cu") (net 2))
 (segment (start 97.8 107.945) (end 94.62 107.945) (width 0.25) (layer "B.Cu") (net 2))
 (segment (start 111.125 113.665) (end 108.585 113.665) (width 0.25) (layer "B.Cu") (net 29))
 (segment (start 107.955 118.105) (end 108.585 117.475) (width 0.25) (layer "B.Cu") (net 29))
 (segment (start 108.585 113.665) (end 107.945 113.025) (width 0.25) (layer "B.Cu") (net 29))
 (segment (start 105.42 118.105) (end 107.955 118.105) (width 0.25) (layer "B.Cu") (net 29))
 (segment (start 107.945 113.025) (end 105.42 113.025) (width 0.25) (layer "B.Cu") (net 29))
 (segment (start 108.585 117.475) (end 108.585 113.665) (width 0.25) (layer "B.Cu") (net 29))
 (segment (start 82.55 121.285) (end 82.55 117.475) (width 0.25) (layer "B.Cu") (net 19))
 (segment (start 80.01 123.825) (end 82.55 121.285) (width 0.25) (layer "B.Cu") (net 19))
 (segment (start 82.55 117.475) (end 83.185 116.84) (width 0.25) (layer "B.Cu") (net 19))
 (segment (start 83.185 116.84) (end 85.885 116.84) (width 0.25) (layer "B.Cu") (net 19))
 (segment (start 80.01 125.095) (end 80.01 123.825) (width 0.25) (layer "B.Cu") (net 19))
 (segment (start 92.075 132.08) (end 92.075 127) (width 0.25) (layer "B.Cu") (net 6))
 (segment (start 92.075 127) (end 91.44 126.365) (width 0.25) (layer "B.Cu") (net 6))
 (segment (start 86.995 119.38) (end 85.885 119.38) (width 0.25) (layer "B.Cu") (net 18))
 (segment (start 91.44 123.825) (end 86.995 119.38) (width 0.25) (layer "B.Cu") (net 18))
 (segment (start 101.6 111.76) (end 101.6 114.935) (width 0.25) (layer "B.Cu") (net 30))
 (segment (start 101.6 114.935) (end 102.23 115.565) (width 0.25) (layer "B.Cu") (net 30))
 (segment (start 102.875 110.485) (end 101.6 111.76) (width 0.25) (layer "B.Cu") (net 30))
 (segment (start 105.42 110.485) (end 102.875 110.485) (width 0.25) (layer "B.Cu") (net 30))
 (segment (start 102.23 115.565) (end 105.42 115.565) (width 0.25) (layer "B.Cu") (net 30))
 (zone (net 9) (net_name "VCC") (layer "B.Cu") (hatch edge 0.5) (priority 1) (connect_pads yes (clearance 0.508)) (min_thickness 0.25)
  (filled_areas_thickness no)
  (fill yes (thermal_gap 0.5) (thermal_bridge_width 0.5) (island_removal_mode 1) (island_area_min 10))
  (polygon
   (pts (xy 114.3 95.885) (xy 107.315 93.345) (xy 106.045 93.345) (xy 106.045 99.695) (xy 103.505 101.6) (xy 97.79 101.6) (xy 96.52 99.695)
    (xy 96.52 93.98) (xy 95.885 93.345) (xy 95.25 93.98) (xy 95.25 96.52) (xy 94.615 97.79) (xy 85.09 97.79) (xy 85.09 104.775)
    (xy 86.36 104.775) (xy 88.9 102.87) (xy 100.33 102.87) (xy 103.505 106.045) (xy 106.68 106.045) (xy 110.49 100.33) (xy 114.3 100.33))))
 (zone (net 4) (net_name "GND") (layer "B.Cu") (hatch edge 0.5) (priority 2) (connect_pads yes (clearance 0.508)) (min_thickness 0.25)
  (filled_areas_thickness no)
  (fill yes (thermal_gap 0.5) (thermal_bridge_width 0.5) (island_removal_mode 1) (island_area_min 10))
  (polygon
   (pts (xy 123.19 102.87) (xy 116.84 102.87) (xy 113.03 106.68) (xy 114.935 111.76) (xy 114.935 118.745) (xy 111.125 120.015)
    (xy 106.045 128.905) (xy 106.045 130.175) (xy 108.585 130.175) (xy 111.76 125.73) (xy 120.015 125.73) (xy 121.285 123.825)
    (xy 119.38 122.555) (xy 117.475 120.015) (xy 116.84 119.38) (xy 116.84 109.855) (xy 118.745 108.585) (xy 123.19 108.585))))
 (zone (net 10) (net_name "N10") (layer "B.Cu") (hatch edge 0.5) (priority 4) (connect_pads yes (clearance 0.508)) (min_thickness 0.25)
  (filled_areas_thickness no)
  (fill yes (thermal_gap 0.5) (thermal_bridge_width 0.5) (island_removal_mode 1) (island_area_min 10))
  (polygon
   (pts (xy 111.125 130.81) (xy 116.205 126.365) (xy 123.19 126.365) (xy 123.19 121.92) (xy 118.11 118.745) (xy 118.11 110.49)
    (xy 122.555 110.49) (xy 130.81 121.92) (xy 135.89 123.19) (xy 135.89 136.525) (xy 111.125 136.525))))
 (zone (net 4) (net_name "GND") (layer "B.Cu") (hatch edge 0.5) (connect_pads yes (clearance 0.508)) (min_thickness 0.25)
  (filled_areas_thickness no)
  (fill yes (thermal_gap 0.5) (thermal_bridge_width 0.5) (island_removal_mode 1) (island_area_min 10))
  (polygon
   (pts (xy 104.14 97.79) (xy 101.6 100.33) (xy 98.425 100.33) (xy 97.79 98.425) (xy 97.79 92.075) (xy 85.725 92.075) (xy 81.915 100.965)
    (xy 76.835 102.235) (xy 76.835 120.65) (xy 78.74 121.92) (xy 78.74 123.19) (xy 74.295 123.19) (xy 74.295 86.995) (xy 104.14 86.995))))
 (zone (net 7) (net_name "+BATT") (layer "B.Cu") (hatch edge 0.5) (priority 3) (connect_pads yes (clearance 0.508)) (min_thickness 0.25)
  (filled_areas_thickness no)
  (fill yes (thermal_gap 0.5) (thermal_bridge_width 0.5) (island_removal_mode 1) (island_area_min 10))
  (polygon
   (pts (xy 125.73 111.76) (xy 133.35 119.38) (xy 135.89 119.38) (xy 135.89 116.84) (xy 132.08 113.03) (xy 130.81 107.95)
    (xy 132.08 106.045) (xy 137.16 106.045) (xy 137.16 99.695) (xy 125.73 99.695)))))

